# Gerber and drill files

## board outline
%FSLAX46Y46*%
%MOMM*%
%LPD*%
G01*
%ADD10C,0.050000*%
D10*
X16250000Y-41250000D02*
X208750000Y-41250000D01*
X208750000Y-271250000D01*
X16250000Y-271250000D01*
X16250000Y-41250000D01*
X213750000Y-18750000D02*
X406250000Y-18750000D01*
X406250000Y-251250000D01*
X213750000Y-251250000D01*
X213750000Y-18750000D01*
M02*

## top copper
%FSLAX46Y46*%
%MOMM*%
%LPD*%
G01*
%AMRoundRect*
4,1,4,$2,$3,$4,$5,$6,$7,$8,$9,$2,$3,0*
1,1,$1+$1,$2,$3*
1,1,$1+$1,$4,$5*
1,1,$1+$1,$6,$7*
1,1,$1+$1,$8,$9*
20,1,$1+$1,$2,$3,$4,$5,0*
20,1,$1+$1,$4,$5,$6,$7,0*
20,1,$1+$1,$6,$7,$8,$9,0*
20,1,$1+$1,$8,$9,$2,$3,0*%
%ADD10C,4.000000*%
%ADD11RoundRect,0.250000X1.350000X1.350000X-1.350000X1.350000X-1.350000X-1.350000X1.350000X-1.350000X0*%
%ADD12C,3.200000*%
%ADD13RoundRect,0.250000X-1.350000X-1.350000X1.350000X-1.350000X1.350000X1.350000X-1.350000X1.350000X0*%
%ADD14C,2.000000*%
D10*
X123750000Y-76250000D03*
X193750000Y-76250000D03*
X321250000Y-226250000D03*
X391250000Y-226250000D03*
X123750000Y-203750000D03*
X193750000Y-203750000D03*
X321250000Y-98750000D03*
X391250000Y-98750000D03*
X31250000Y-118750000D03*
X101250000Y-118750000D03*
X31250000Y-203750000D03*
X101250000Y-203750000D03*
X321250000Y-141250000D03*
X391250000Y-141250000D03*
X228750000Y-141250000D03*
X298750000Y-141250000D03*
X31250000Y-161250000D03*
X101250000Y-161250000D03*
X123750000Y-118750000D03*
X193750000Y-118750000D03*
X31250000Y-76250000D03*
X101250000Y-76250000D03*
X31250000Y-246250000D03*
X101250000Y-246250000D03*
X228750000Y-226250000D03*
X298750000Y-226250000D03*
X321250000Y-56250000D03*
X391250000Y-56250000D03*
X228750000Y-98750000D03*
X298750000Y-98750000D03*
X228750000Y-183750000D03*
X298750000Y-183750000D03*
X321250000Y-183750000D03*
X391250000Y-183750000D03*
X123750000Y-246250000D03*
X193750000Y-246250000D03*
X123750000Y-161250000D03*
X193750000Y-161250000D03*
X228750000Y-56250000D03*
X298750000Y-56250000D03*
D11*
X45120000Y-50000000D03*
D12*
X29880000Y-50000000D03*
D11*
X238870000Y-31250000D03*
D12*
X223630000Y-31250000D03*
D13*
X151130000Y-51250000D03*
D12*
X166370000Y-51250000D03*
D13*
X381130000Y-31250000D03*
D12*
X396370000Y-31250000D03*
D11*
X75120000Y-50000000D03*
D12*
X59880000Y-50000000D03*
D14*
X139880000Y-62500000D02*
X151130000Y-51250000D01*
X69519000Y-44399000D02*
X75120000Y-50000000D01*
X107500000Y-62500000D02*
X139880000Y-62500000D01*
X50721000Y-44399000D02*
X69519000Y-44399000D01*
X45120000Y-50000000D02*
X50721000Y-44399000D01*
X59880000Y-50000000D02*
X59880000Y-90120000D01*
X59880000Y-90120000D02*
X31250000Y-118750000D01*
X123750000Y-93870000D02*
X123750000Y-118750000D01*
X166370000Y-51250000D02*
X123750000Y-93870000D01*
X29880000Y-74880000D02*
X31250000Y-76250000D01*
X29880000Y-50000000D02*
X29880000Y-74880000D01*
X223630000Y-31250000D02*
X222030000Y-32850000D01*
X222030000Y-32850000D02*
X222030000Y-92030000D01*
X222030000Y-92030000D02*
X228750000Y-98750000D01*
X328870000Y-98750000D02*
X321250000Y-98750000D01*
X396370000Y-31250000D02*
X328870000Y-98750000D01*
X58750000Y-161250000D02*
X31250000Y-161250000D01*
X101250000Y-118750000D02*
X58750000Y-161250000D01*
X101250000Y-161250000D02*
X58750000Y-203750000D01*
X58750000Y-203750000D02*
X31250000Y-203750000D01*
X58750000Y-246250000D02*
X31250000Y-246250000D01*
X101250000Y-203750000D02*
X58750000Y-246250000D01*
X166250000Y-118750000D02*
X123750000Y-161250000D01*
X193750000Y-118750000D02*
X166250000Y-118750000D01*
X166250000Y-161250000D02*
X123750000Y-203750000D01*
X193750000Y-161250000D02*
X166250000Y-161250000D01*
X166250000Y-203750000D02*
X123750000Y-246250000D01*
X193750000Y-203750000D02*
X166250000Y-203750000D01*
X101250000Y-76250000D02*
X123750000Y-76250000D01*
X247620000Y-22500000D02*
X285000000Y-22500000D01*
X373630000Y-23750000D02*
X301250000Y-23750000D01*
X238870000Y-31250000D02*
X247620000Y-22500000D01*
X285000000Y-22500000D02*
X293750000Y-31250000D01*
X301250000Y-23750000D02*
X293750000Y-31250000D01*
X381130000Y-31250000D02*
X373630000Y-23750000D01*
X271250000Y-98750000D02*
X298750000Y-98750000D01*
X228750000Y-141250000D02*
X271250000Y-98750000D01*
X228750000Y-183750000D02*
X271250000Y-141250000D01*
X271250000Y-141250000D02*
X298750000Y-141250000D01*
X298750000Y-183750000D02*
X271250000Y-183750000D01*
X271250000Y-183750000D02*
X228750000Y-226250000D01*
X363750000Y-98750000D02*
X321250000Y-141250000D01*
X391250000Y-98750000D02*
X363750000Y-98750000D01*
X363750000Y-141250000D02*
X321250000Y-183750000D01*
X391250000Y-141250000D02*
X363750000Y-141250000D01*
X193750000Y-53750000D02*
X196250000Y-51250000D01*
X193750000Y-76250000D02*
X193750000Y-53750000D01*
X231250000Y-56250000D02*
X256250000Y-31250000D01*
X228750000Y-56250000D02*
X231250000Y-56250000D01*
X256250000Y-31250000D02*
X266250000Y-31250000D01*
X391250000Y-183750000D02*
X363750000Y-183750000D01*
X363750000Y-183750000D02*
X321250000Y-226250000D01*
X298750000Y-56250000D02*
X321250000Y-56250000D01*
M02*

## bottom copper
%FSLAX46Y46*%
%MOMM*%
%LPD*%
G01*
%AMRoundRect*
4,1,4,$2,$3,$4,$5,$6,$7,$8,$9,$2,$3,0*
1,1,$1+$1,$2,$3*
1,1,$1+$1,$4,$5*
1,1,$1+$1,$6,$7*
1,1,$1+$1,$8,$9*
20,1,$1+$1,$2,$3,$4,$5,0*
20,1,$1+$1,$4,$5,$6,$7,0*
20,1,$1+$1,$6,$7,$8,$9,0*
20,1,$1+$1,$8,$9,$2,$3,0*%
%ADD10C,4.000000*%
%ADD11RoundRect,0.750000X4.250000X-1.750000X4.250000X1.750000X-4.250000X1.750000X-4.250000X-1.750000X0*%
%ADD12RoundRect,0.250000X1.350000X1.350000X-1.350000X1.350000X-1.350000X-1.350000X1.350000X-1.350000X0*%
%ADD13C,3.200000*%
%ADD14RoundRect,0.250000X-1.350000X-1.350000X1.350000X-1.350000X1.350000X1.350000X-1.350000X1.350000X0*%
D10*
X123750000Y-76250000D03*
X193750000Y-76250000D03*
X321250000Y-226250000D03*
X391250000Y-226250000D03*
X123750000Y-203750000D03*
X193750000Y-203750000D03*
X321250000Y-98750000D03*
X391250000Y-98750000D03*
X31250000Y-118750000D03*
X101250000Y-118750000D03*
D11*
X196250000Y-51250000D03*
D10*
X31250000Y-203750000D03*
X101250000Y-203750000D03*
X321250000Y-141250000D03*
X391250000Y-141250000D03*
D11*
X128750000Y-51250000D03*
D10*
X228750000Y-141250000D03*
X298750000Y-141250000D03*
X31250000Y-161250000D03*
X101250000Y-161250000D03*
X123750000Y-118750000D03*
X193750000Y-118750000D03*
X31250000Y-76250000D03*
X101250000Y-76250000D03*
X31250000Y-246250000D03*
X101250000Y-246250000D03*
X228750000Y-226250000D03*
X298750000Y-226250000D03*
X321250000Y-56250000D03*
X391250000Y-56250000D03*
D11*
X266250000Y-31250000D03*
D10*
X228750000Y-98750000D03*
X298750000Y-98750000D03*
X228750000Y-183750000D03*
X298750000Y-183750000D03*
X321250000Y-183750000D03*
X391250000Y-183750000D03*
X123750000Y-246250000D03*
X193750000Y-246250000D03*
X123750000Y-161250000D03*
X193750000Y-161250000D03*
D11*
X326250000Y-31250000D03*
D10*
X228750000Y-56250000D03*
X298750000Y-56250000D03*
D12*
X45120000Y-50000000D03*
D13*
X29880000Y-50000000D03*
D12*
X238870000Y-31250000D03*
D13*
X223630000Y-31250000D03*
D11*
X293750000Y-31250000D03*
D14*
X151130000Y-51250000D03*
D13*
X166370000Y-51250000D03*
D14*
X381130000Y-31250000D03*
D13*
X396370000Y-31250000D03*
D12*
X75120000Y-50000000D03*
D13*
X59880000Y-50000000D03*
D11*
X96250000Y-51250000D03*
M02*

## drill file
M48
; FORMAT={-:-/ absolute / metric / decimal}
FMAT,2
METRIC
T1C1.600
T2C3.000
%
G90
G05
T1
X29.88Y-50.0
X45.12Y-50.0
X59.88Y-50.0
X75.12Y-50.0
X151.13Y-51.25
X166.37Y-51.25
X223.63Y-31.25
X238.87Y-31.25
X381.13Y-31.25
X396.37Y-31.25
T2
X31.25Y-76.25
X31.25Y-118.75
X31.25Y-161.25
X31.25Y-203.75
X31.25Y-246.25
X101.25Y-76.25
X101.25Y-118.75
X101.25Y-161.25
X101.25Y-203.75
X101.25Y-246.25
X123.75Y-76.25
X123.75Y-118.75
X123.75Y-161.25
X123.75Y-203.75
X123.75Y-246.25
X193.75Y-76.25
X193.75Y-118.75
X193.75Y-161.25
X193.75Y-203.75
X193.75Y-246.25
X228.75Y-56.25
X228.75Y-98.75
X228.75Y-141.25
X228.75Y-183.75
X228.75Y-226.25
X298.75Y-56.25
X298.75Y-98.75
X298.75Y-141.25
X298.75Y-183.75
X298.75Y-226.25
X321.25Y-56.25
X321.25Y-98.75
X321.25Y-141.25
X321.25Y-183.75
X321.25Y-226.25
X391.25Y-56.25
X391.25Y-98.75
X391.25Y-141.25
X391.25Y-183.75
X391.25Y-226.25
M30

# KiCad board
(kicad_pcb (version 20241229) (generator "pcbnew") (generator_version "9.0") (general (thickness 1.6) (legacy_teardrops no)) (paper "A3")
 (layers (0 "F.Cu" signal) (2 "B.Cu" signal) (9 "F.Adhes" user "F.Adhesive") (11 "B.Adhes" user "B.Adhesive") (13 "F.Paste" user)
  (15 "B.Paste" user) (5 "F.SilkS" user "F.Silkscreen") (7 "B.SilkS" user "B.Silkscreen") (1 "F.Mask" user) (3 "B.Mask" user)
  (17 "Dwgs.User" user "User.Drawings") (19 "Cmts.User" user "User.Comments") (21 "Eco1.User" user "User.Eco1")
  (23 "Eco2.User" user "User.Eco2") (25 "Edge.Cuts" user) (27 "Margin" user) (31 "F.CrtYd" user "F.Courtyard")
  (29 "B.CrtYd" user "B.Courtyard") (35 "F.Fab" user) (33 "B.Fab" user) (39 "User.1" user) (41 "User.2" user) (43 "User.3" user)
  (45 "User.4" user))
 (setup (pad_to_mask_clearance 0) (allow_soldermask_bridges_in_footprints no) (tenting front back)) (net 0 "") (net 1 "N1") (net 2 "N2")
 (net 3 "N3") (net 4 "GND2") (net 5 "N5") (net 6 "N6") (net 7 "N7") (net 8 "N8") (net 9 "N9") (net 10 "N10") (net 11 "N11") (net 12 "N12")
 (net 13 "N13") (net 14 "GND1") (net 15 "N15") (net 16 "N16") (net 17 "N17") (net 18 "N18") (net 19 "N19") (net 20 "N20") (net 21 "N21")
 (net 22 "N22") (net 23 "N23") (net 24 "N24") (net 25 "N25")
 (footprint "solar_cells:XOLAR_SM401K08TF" (layer "F.Cu") (at 158.75 76.25)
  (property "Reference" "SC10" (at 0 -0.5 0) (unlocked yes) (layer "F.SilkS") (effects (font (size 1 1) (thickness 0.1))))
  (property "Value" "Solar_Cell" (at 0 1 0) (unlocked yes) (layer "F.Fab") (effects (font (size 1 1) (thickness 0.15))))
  (pad "1" thru_hole circle (at -35 0) (size 4 4) (drill 3) (layers "*.Cu" "*.Mask") (remove_unused_layers no) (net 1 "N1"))
  (pad "2" thru_hole circle (at 35 0) (size 4 4) (drill 3) (layers "*.Cu" "*.Mask") (remove_unused_layers no) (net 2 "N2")))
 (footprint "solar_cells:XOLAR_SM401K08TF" (layer "F.Cu") (at 356.25 226.25)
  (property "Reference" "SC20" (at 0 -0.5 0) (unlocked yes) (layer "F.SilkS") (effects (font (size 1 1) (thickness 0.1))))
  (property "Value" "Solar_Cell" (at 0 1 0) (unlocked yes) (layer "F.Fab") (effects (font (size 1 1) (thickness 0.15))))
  (pad "1" thru_hole circle (at -35 0) (size 4 4) (drill 3) (layers "*.Cu" "*.Mask") (remove_unused_layers no) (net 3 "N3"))
  (pad "2" thru_hole circle (at 35 0) (size 4 4) (drill 3) (layers "*.Cu" "*.Mask") (remove_unused_layers no) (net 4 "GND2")))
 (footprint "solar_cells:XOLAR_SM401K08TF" (layer "F.Cu") (at 158.75 203.75)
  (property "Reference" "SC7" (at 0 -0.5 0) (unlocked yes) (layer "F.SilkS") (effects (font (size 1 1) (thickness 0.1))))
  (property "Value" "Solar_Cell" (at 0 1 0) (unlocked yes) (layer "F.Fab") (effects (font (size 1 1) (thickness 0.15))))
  (pad "1" thru_hole circle (at -35 0) (size 4 4) (drill 3) (layers "*.Cu" "*.Mask") (remove_unused_layers no) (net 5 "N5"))
  (pad "2" thru_hole circle (at 35 0) (size 4 4) (drill 3) (layers "*.Cu" "*.Mask") (remove_unused_layers no) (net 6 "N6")))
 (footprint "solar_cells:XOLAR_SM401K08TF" (layer "F.Cu") (at 356.25 98.75)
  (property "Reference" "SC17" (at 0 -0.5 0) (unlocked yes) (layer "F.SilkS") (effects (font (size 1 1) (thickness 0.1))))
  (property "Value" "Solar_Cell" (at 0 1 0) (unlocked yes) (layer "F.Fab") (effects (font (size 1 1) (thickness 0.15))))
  (pad "1" thru_hole circle (at -35 0) (size 4 4) (drill 3) (layers "*.Cu" "*.Mask") (remove_unused_layers no) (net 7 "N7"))
  (pad "2" thru_hole circle (at 35 0) (size 4 4) (drill 3) (layers "*.Cu" "*.Mask") (remove_unused_layers no) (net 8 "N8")))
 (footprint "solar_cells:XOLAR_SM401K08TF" (layer "F.Cu") (at 66.25 118.75)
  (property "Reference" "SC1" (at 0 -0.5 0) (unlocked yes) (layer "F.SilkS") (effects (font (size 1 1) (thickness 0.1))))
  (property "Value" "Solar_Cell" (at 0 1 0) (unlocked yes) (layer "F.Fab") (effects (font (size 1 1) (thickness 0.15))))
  (pad "1" thru_hole circle (at -35 0) (size 4 4) (drill 3) (layers "*.Cu" "*.Mask") (remove_unused_layers no) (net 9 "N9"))
  (pad "2" thru_hole circle (at 35 0) (size 4 4) (drill 3) (layers "*.Cu" "*.Mask") (remove_unused_layers no) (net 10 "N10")))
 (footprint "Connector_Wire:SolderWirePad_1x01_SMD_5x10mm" (layer "F.Cu") (at 196.25 51.25 90)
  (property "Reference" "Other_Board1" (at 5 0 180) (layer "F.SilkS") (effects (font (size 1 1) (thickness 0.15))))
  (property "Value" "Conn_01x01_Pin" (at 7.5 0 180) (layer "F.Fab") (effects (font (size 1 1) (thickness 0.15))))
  (pad "1" smd roundrect (at 0 0 90) (size 5 10) (layers "F.Mask" "B.Cu" "F.Paste") (roundrect_rratio 0.15) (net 2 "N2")))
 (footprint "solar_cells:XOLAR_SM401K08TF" (layer "F.Cu") (at 66.25 203.75)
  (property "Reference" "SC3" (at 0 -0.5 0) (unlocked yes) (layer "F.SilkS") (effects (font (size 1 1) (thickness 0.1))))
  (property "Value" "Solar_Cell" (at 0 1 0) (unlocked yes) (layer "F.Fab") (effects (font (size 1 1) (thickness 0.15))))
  (pad "1" thru_hole circle (at -35 0) (size 4 4) (drill 3) (layers "*.Cu" "*.Mask") (remove_unused_layers no) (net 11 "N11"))
  (pad "2" thru_hole circle (at 35 0) (size 4 4) (drill 3) (layers "*.Cu" "*.Mask") (remove_unused_layers no) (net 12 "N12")))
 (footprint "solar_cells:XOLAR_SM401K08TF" (layer "F.Cu") (at 356.25 141.25)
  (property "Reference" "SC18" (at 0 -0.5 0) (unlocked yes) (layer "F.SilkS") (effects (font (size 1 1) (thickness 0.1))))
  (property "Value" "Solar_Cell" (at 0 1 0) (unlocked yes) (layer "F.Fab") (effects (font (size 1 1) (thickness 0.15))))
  (pad "1" thru_hole circle (at -35 0) (size 4 4) (drill 3) (layers "*.Cu" "*.Mask") (remove_unused_layers no) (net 8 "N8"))
  (pad "2" thru_hole circle (at 35 0) (size 4 4) (drill 3) (layers "*.Cu" "*.Mask") (remove_unused_layers no) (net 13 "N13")))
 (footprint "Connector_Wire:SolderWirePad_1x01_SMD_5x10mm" (layer "F.Cu") (at 128.75 51.25 90)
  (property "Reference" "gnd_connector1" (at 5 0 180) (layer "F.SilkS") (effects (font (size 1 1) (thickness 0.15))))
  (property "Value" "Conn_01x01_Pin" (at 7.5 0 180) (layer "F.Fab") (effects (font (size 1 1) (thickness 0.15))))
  (pad "1" smd roundrect (at 0 0 90) (size 5 10) (layers "F.Mask" "B.Cu" "F.Paste") (roundrect_rratio 0.15) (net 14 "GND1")))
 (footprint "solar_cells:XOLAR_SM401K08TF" (layer "F.Cu") (at 263.75 141.25)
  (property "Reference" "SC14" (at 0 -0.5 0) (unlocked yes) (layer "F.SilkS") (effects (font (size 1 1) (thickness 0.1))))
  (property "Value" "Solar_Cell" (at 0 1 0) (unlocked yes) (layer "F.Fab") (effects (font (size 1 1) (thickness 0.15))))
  (pad "1" thru_hole circle (at -35 0) (size 4 4) (drill 3) (layers "*.Cu" "*.Mask") (remove_unused_layers no) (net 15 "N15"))
  (pad "2" thru_hole circle (at 35 0) (size 4 4) (drill 3) (layers "*.Cu" "*.Mask") (remove_unused_layers no) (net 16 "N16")))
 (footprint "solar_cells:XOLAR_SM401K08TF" (layer "F.Cu") (at 66.25 161.25)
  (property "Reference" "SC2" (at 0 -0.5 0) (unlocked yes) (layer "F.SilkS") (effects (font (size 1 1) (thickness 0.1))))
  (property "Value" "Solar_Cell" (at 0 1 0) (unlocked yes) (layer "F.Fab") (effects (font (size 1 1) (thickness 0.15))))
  (pad "1" thru_hole circle (at -35 0) (size 4 4) (drill 3) (layers "*.Cu" "*.Mask") (remove_unused_layers no) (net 10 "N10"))
  (pad "2" thru_hole circle (at 35 0) (size 4 4) (drill 3) (layers "*.Cu" "*.Mask") (remove_unused_layers no) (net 11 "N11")))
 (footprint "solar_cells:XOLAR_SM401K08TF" (layer "F.Cu") (at 158.75 118.75)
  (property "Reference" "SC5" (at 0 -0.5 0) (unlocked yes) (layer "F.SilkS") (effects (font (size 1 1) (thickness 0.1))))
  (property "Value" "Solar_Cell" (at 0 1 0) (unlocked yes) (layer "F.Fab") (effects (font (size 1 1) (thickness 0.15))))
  (pad "1" thru_hole circle (at -35 0) (size 4 4) (drill 3) (layers "*.Cu" "*.Mask") (remove_unused_layers no) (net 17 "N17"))
  (pad "2" thru_hole circle (at 35 0) (size 4 4) (drill 3) (layers "*.Cu" "*.Mask") (remove_unused_layers no) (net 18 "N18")))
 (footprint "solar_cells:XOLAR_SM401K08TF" (layer "F.Cu") (at 66.25 76.25)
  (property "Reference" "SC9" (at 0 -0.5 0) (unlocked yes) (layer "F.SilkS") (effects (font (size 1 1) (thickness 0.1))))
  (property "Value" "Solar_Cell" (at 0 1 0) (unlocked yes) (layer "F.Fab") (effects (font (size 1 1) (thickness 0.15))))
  (pad "1" thru_hole circle (at -35 0) (size 4 4) (drill 3) (layers "*.Cu" "*.Mask") (remove_unused_layers no) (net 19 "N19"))
  (pad "2" thru_hole circle (at 35 0) (size 4 4) (drill 3) (layers "*.Cu" "*.Mask") (remove_unused_layers no) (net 1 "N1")))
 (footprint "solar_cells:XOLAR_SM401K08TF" (layer "F.Cu") (at 66.25 246.25)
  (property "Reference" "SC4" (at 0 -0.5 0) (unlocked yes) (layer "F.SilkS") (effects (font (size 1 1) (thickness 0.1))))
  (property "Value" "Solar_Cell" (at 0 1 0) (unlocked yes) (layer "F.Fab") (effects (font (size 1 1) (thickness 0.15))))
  (pad "1" thru_hole circle (at -35 0) (size 4 4) (drill 3) (layers "*.Cu" "*.Mask") (remove_unused_layers no) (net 12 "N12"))
  (pad "2" thru_hole circle (at 35 0) (size 4 4) (drill 3) (layers "*.Cu" "*.Mask") (remove_unused_layers no) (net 14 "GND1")))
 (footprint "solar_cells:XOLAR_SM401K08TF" (layer "F.Cu") (at 263.75 226.25)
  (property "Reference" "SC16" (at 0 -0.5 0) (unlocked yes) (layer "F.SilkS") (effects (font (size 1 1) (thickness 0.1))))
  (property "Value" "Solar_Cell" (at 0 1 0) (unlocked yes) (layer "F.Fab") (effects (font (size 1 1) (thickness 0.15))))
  (pad "1" thru_hole circle (at -35 0) (size 4 4) (drill 3) (layers "*.Cu" "*.Mask") (remove_unused_layers no) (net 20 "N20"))
  (pad "2" thru_hole circle (at 35 0) (size 4 4) (drill 3) (layers "*.Cu" "*.Mask") (remove_unused_layers no) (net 4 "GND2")))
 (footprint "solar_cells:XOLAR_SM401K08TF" (layer "F.Cu") (at 356.25 56.25)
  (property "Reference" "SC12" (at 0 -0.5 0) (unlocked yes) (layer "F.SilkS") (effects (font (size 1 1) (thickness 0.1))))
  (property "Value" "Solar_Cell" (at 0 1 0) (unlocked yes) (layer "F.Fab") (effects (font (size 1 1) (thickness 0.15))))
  (pad "1" thru_hole circle (at -35 0) (size 4 4) (drill 3) (layers "*.Cu" "*.Mask") (remove_unused_layers no) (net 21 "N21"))
  (pad "2" thru_hole circle (at 35 0) (size 4 4) (drill 3) (layers "*.Cu" "*.Mask") (remove_unused_layers no) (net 4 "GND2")))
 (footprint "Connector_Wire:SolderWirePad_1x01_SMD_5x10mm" (layer "F.Cu") (at 266.25 31.25 90)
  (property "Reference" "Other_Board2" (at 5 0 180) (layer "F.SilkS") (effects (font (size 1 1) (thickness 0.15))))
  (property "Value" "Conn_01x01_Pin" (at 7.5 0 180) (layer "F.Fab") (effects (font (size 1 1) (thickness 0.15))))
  (pad "1" smd roundrect (at 0 0 90) (size 5 10) (layers "F.Mask" "B.Cu" "F.Paste") (roundrect_rratio 0.15) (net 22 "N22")))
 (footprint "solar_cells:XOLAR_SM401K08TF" (layer "F.Cu") (at 263.75 98.75)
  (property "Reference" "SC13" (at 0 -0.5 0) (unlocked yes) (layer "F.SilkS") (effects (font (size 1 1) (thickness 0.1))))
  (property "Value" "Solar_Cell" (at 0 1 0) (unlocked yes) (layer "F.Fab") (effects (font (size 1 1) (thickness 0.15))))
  (pad "1" thru_hole circle (at -35 0) (size 4 4) (drill 3) (layers "*.Cu" "*.Mask") (remove_unused_layers no) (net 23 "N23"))
  (pad "2" thru_hole circle (at 35 0) (size 4 4) (drill 3) (layers "*.Cu" "*.Mask") (remove_unused_layers no) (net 15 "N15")))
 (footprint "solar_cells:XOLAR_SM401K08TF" (layer "F.Cu") (at 263.75 183.75)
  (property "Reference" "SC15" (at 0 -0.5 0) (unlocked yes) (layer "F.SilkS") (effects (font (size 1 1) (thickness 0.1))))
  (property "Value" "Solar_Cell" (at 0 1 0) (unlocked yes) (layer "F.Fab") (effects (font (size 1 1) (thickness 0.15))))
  (pad "1" thru_hole circle (at -35 0) (size 4 4) (drill 3) (layers "*.Cu" "*.Mask") (remove_unused_layers no) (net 16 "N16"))
  (pad "2" thru_hole circle (at 35 0) (size 4 4) (drill 3) (layers "*.Cu" "*.Mask") (remove_unused_layers no) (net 20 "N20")))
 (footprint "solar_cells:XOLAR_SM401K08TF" (layer "F.Cu") (at 356.25 183.75)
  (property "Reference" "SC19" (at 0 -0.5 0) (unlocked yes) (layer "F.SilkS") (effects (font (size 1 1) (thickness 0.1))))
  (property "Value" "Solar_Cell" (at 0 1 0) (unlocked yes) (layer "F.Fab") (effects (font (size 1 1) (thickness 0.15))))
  (pad "1" thru_hole circle (at -35 0) (size 4 4) (drill 3) (layers "*.Cu" "*.Mask") (remove_unused_layers no) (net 13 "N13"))
  (pad "2" thru_hole circle (at 35 0) (size 4 4) (drill 3) (layers "*.Cu" "*.Mask") (remove_unused_layers no) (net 3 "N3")))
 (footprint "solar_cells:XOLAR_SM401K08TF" (layer "F.Cu") (at 158.75 246.25)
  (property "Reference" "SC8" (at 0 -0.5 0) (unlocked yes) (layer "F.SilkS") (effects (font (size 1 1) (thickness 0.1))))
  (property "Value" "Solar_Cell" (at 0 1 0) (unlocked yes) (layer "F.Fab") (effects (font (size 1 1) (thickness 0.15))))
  (pad "1" thru_hole circle (at -35 0) (size 4 4) (drill 3) (layers "*.Cu" "*.Mask") (remove_unused_layers no) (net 6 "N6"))
  (pad "2" thru_hole circle (at 35 0) (size 4 4) (drill 3) (layers "*.Cu" "*.Mask") (remove_unused_layers no) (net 14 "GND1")))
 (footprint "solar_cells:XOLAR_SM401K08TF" (layer "F.Cu") (at 158.75 161.25)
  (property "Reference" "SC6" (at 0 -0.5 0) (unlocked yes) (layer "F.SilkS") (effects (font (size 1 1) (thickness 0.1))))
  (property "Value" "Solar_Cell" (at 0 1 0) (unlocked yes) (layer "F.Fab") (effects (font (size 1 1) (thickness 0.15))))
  (pad "1" thru_hole circle (at -35 0) (size 4 4) (drill 3) (layers "*.Cu" "*.Mask") (remove_unused_layers no) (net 18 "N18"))
  (pad "2" thru_hole circle (at 35 0) (size 4 4) (drill 3) (layers "*.Cu" "*.Mask") (remove_unused_layers no) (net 5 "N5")))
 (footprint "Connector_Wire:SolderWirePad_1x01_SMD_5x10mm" (layer "F.Cu") (at 326.25 31.25 90)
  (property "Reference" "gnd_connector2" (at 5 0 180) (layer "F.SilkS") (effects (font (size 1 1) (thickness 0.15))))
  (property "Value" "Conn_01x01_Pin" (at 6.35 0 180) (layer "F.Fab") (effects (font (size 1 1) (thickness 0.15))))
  (pad "1" smd roundrect (at 0 0 90) (size 5 10) (layers "F.Mask" "B.Cu" "F.Paste") (roundrect_rratio 0.15) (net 4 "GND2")))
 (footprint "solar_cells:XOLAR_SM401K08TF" (layer "F.Cu") (at 263.75 56.25)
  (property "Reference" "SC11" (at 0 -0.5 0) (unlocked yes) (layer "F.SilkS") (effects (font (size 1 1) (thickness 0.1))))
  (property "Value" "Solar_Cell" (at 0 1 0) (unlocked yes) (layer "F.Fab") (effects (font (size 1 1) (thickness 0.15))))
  (pad "1" thru_hole circle (at -35 0) (size 4 4) (drill 3) (layers "*.Cu" "*.Mask") (remove_unused_layers no) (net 22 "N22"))
  (pad "2" thru_hole circle (at 35 0) (size 4 4) (drill 3) (layers "*.Cu" "*.Mask") (remove_unused_layers no) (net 21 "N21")))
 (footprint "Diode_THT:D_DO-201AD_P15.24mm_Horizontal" (layer "B.Cu") (at 45.12 50 180)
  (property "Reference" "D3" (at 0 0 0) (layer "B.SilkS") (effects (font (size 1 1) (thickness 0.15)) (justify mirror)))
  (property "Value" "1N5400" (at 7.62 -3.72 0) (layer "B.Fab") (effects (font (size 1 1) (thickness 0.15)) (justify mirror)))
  (pad "1" thru_hole roundrect (at 0 0 180) (size 3.2 3.2) (drill 1.6) (layers "*.Cu" "*.Mask") (remove_unused_layers no)
   (roundrect_rratio 0.078125) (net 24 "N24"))
  (pad "2" thru_hole circle (at 15.24 0 180) (size 3.2 3.2) (drill 1.6) (layers "*.Cu" "*.Mask") (remove_unused_layers no) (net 19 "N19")))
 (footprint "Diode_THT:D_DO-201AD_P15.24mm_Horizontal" (layer "B.Cu") (at 238.87 31.25 180)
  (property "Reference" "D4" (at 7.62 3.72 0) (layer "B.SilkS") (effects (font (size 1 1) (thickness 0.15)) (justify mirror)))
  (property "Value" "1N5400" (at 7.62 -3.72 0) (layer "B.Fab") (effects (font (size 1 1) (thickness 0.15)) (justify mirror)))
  (pad "1" thru_hole roundrect (at 0 0 180) (size 3.2 3.2) (drill 1.6) (layers "*.Cu" "*.Mask") (remove_unused_layers no)
   (roundrect_rratio 0.078125) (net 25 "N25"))
  (pad "2" thru_hole circle (at 15.24 0 180) (size 3.2 3.2) (drill 1.6) (layers "*.Cu" "*.Mask") (remove_unused_layers no) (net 23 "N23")))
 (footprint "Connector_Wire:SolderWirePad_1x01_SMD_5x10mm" (layer "B.Cu") (at 293.75 31.25 90)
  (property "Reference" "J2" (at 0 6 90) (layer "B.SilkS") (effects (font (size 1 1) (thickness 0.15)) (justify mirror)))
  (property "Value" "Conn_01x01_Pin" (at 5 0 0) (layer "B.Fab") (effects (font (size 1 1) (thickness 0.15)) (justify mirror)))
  (pad "1" smd roundrect (at 0 0 90) (size 5 10) (layers "F.Mask" "B.Cu" "F.Paste") (roundrect_rratio 0.15) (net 25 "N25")))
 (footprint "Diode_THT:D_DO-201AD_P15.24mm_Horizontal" (layer "B.Cu") (at 151.13 51.25)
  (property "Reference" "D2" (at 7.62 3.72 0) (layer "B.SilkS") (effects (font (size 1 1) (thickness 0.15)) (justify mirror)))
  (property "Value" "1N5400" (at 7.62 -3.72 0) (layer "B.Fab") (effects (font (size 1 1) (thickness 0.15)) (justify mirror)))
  (pad "1" thru_hole roundrect (at 0 0) (size 3.2 3.2) (drill 1.6) (layers "*.Cu" "*.Mask") (remove_unused_layers no)
   (roundrect_rratio 0.078125) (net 24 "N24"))
  (pad "2" thru_hole circle (at 15.24 0) (size 3.2 3.2) (drill 1.6) (layers "*.Cu" "*.Mask") (remove_unused_layers no) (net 17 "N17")))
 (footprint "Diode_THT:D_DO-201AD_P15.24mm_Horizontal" (layer "B.Cu") (at 381.13 31.25)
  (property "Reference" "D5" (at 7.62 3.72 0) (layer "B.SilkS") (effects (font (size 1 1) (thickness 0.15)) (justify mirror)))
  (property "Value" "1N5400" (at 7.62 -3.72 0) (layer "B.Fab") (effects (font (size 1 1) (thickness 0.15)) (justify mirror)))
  (pad "1" thru_hole roundrect (at 0 0) (size 3.2 3.2) (drill 1.6) (layers "*.Cu" "*.Mask") (remove_unused_layers no)
   (roundrect_rratio 0.078125) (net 25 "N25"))
  (pad "2" thru_hole circle (at 15.24 0) (size 3.2 3.2) (drill 1.6) (layers "*.Cu" "*.Mask") (remove_unused_layers no) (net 7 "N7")))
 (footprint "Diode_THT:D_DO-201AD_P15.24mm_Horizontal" (layer "B.Cu") (at 75.12 50 180)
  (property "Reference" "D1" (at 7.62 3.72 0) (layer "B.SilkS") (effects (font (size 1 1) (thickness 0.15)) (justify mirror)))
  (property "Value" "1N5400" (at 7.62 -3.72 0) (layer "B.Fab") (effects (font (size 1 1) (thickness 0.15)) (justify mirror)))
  (pad "1" thru_hole roundrect (at 0 0 180) (size 3.2 3.2) (drill 1.6) (layers "*.Cu" "*.Mask") (remove_unused_layers no)
   (roundrect_rratio 0.078125) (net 24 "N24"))
  (pad "2" thru_hole circle (at 15.24 0 180) (size 3.2 3.2) (drill 1.6) (layers "*.Cu" "*.Mask") (remove_unused_layers no) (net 9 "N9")))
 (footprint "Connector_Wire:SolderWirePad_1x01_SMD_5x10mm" (layer "B.Cu") (at 96.25 51.25 90)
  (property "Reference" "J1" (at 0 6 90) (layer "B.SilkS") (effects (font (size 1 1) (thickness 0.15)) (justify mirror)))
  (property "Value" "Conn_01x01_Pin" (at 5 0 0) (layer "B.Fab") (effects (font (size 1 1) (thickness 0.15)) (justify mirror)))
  (pad "1" smd roundrect (at 0 0 90) (size 5 10) (layers "F.Mask" "B.Cu" "F.Paste") (roundrect_rratio 0.15) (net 24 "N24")))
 (gr_rect (start 16.25 41.25) (end 208.75 271.25) (stroke (width 0.05) (type default)) (fill no) (layer "Edge.Cuts"))
 (gr_rect (start 213.75 18.75) (end 406.25 251.25) (stroke (width 0.05) (type default)) (fill no) (layer "Edge.Cuts"))
 (segment (start 139.88 62.5) (end 151.13 51.25) (width 2) (layer "F.Cu") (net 24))
 (segment (start 69.519 44.399) (end 75.12 50) (width 2) (layer "F.Cu") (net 24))
 (segment (start 107.5 62.5) (end 139.88 62.5) (width 2) (layer "F.Cu") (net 24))
 (segment (start 50.721 44.399) (end 69.519 44.399) (width 2) (layer "F.Cu") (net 24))
 (segment (start 45.12 50) (end 50.721 44.399) (width 2) (layer "F.Cu") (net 24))
 (segment (start 59.88 50) (end 59.88 90.12) (width 2) (layer "F.Cu") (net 9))
 (segment (start 59.88 90.12) (end 31.25 118.75) (width 2) (layer "F.Cu") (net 9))
 (segment (start 123.75 93.87) (end 123.75 118.75) (width 2) (layer "F.Cu") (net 17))
 (segment (start 166.37 51.25) (end 123.75 93.87) (width 2) (layer "F.Cu") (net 17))
 (segment (start 29.88 74.88) (end 31.25 76.25) (width 2) (layer "F.Cu") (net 19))
 (segment (start 29.88 50) (end 29.88 74.88) (width 2) (layer "F.Cu") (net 19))
 (segment (start 223.63 31.25) (end 222.03 32.85) (width 2) (layer "F.Cu") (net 23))
 (segment (start 222.03 32.85) (end 222.03 92.03) (width 2) (layer "F.Cu") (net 23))
 (segment (start 222.03 92.03) (end 228.75 98.75) (width 2) (layer "F.Cu") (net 23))
 (segment (start 328.87 98.75) (end 321.25 98.75) (width 2) (layer "F.Cu") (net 7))
 (segment (start 396.37 31.25) (end 328.87 98.75) (width 2) (layer "F.Cu") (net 7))
 (segment (start 58.75 161.25) (end 31.25 161.25) (width 2) (layer "F.Cu") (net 10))
 (segment (start 101.25 118.75) (end 58.75 161.25) (width 2) (layer "F.Cu") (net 10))
 (segment (start 101.25 161.25) (end 58.75 203.75) (width 2) (layer "F.Cu") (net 11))
 (segment (start 58.75 203.75) (end 31.25 203.75) (width 2) (layer "F.Cu") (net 11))
 (segment (start 58.75 246.25) (end 31.25 246.25) (width 2) (layer "F.Cu") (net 12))
 (segment (start 101.25 203.75) (end 58.75 246.25) (width 2) (layer "F.Cu") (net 12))
 (segment (start 166.25 118.75) (end 123.75 161.25) (width 2) (layer "F.Cu") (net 18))
 (segment (start 193.75 118.75) (end 166.25 118.75) (width 2) (layer "F.Cu") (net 18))
 (segment (start 166.25 161.25) (end 123.75 203.75) (width 2) (layer "F.Cu") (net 5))
 (segment (start 193.75 161.25) (end 166.25 161.25) (width 2) (layer "F.Cu") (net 5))
 (segment (start 166.25 203.75) (end 123.75 246.25) (width 2) (layer "F.Cu") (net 6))
 (segment (start 193.75 203.75) (end 166.25 203.75) (width 2) (layer "F.Cu") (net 6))
 (segment (start 101.25 76.25) (end 123.75 76.25) (width 2) (layer "F.Cu") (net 1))
 (segment (start 247.62 22.5) (end 285 22.5) (width 2) (layer "F.Cu") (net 25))
 (segment (start 373.63 23.75) (end 301.25 23.75) (width 2) (layer "F.Cu") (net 25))
 (segment (start 238.87 31.25) (end 247.62 22.5) (width 2) (layer "F.Cu") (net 25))
 (segment (start 285 22.5) (end 293.75 31.25) (width 2) (layer "F.Cu") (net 25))
 (segment (start 301.25 23.75) (end 293.75 31.25) (width 2) (layer "F.Cu") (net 25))
 (segment (start 381.13 31.25) (end 373.63 23.75) (width 2) (layer "F.Cu") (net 25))
 (segment (start 271.25 98.75) (end 298.75 98.75) (width 2) (layer "F.Cu") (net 15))
 (segment (start 228.75 141.25) (end 271.25 98.75) (width 2) (layer "F.Cu") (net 15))
 (segment (start 228.75 183.75) (end 271.25 141.25) (width 2) (layer "F.Cu") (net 16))
 (segment (start 271.25 141.25) (end 298.75 141.25) (width 2) (layer "F.Cu") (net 16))
 (segment (start 298.75 183.75) (end 271.25 183.75) (width 2) (layer "F.Cu") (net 20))
 (segment (start 271.25 183.75) (end 228.75 226.25) (width 2) (layer "F.Cu") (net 20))
 (segment (start 363.75 98.75) (end 321.25 141.25) (width 2) (layer "F.Cu") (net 8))
 (segment (start 391.25 98.75) (end 363.75 98.75) (width 2) (layer "F.Cu") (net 8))
 (segment (start 363.75 141.25) (end 321.25 183.75) (width 2) (layer "F.Cu") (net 13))
 (segment (start 391.25 141.25) (end 363.75 141.25) (width 2) (layer "F.Cu") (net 13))
 (segment (start 193.75 53.75) (end 196.25 51.25) (width 2) (layer "F.Cu") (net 2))
 (segment (start 193.75 76.25) (end 193.75 53.75) (width 2) (layer "F.Cu") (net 2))
 (segment (start 231.25 56.25) (end 256.25 31.25) (width 2) (layer "F.Cu") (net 22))
 (segment (start 228.75 56.25) (end 231.25 56.25) (width 2) (layer "F.Cu") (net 22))
 (segment (start 256.25 31.25) (end 266.25 31.25) (width 2) (layer "F.Cu") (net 22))
 (segment (start 391.25 183.75) (end 363.75 183.75) (width 2) (layer "F.Cu") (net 3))
 (segment (start 363.75 183.75) (end 321.25 226.25) (width 2) (layer "F.Cu") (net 3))
 (segment (start 298.75 56.25) (end 321.25 56.25) (width 2) (layer "F.Cu") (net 21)))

